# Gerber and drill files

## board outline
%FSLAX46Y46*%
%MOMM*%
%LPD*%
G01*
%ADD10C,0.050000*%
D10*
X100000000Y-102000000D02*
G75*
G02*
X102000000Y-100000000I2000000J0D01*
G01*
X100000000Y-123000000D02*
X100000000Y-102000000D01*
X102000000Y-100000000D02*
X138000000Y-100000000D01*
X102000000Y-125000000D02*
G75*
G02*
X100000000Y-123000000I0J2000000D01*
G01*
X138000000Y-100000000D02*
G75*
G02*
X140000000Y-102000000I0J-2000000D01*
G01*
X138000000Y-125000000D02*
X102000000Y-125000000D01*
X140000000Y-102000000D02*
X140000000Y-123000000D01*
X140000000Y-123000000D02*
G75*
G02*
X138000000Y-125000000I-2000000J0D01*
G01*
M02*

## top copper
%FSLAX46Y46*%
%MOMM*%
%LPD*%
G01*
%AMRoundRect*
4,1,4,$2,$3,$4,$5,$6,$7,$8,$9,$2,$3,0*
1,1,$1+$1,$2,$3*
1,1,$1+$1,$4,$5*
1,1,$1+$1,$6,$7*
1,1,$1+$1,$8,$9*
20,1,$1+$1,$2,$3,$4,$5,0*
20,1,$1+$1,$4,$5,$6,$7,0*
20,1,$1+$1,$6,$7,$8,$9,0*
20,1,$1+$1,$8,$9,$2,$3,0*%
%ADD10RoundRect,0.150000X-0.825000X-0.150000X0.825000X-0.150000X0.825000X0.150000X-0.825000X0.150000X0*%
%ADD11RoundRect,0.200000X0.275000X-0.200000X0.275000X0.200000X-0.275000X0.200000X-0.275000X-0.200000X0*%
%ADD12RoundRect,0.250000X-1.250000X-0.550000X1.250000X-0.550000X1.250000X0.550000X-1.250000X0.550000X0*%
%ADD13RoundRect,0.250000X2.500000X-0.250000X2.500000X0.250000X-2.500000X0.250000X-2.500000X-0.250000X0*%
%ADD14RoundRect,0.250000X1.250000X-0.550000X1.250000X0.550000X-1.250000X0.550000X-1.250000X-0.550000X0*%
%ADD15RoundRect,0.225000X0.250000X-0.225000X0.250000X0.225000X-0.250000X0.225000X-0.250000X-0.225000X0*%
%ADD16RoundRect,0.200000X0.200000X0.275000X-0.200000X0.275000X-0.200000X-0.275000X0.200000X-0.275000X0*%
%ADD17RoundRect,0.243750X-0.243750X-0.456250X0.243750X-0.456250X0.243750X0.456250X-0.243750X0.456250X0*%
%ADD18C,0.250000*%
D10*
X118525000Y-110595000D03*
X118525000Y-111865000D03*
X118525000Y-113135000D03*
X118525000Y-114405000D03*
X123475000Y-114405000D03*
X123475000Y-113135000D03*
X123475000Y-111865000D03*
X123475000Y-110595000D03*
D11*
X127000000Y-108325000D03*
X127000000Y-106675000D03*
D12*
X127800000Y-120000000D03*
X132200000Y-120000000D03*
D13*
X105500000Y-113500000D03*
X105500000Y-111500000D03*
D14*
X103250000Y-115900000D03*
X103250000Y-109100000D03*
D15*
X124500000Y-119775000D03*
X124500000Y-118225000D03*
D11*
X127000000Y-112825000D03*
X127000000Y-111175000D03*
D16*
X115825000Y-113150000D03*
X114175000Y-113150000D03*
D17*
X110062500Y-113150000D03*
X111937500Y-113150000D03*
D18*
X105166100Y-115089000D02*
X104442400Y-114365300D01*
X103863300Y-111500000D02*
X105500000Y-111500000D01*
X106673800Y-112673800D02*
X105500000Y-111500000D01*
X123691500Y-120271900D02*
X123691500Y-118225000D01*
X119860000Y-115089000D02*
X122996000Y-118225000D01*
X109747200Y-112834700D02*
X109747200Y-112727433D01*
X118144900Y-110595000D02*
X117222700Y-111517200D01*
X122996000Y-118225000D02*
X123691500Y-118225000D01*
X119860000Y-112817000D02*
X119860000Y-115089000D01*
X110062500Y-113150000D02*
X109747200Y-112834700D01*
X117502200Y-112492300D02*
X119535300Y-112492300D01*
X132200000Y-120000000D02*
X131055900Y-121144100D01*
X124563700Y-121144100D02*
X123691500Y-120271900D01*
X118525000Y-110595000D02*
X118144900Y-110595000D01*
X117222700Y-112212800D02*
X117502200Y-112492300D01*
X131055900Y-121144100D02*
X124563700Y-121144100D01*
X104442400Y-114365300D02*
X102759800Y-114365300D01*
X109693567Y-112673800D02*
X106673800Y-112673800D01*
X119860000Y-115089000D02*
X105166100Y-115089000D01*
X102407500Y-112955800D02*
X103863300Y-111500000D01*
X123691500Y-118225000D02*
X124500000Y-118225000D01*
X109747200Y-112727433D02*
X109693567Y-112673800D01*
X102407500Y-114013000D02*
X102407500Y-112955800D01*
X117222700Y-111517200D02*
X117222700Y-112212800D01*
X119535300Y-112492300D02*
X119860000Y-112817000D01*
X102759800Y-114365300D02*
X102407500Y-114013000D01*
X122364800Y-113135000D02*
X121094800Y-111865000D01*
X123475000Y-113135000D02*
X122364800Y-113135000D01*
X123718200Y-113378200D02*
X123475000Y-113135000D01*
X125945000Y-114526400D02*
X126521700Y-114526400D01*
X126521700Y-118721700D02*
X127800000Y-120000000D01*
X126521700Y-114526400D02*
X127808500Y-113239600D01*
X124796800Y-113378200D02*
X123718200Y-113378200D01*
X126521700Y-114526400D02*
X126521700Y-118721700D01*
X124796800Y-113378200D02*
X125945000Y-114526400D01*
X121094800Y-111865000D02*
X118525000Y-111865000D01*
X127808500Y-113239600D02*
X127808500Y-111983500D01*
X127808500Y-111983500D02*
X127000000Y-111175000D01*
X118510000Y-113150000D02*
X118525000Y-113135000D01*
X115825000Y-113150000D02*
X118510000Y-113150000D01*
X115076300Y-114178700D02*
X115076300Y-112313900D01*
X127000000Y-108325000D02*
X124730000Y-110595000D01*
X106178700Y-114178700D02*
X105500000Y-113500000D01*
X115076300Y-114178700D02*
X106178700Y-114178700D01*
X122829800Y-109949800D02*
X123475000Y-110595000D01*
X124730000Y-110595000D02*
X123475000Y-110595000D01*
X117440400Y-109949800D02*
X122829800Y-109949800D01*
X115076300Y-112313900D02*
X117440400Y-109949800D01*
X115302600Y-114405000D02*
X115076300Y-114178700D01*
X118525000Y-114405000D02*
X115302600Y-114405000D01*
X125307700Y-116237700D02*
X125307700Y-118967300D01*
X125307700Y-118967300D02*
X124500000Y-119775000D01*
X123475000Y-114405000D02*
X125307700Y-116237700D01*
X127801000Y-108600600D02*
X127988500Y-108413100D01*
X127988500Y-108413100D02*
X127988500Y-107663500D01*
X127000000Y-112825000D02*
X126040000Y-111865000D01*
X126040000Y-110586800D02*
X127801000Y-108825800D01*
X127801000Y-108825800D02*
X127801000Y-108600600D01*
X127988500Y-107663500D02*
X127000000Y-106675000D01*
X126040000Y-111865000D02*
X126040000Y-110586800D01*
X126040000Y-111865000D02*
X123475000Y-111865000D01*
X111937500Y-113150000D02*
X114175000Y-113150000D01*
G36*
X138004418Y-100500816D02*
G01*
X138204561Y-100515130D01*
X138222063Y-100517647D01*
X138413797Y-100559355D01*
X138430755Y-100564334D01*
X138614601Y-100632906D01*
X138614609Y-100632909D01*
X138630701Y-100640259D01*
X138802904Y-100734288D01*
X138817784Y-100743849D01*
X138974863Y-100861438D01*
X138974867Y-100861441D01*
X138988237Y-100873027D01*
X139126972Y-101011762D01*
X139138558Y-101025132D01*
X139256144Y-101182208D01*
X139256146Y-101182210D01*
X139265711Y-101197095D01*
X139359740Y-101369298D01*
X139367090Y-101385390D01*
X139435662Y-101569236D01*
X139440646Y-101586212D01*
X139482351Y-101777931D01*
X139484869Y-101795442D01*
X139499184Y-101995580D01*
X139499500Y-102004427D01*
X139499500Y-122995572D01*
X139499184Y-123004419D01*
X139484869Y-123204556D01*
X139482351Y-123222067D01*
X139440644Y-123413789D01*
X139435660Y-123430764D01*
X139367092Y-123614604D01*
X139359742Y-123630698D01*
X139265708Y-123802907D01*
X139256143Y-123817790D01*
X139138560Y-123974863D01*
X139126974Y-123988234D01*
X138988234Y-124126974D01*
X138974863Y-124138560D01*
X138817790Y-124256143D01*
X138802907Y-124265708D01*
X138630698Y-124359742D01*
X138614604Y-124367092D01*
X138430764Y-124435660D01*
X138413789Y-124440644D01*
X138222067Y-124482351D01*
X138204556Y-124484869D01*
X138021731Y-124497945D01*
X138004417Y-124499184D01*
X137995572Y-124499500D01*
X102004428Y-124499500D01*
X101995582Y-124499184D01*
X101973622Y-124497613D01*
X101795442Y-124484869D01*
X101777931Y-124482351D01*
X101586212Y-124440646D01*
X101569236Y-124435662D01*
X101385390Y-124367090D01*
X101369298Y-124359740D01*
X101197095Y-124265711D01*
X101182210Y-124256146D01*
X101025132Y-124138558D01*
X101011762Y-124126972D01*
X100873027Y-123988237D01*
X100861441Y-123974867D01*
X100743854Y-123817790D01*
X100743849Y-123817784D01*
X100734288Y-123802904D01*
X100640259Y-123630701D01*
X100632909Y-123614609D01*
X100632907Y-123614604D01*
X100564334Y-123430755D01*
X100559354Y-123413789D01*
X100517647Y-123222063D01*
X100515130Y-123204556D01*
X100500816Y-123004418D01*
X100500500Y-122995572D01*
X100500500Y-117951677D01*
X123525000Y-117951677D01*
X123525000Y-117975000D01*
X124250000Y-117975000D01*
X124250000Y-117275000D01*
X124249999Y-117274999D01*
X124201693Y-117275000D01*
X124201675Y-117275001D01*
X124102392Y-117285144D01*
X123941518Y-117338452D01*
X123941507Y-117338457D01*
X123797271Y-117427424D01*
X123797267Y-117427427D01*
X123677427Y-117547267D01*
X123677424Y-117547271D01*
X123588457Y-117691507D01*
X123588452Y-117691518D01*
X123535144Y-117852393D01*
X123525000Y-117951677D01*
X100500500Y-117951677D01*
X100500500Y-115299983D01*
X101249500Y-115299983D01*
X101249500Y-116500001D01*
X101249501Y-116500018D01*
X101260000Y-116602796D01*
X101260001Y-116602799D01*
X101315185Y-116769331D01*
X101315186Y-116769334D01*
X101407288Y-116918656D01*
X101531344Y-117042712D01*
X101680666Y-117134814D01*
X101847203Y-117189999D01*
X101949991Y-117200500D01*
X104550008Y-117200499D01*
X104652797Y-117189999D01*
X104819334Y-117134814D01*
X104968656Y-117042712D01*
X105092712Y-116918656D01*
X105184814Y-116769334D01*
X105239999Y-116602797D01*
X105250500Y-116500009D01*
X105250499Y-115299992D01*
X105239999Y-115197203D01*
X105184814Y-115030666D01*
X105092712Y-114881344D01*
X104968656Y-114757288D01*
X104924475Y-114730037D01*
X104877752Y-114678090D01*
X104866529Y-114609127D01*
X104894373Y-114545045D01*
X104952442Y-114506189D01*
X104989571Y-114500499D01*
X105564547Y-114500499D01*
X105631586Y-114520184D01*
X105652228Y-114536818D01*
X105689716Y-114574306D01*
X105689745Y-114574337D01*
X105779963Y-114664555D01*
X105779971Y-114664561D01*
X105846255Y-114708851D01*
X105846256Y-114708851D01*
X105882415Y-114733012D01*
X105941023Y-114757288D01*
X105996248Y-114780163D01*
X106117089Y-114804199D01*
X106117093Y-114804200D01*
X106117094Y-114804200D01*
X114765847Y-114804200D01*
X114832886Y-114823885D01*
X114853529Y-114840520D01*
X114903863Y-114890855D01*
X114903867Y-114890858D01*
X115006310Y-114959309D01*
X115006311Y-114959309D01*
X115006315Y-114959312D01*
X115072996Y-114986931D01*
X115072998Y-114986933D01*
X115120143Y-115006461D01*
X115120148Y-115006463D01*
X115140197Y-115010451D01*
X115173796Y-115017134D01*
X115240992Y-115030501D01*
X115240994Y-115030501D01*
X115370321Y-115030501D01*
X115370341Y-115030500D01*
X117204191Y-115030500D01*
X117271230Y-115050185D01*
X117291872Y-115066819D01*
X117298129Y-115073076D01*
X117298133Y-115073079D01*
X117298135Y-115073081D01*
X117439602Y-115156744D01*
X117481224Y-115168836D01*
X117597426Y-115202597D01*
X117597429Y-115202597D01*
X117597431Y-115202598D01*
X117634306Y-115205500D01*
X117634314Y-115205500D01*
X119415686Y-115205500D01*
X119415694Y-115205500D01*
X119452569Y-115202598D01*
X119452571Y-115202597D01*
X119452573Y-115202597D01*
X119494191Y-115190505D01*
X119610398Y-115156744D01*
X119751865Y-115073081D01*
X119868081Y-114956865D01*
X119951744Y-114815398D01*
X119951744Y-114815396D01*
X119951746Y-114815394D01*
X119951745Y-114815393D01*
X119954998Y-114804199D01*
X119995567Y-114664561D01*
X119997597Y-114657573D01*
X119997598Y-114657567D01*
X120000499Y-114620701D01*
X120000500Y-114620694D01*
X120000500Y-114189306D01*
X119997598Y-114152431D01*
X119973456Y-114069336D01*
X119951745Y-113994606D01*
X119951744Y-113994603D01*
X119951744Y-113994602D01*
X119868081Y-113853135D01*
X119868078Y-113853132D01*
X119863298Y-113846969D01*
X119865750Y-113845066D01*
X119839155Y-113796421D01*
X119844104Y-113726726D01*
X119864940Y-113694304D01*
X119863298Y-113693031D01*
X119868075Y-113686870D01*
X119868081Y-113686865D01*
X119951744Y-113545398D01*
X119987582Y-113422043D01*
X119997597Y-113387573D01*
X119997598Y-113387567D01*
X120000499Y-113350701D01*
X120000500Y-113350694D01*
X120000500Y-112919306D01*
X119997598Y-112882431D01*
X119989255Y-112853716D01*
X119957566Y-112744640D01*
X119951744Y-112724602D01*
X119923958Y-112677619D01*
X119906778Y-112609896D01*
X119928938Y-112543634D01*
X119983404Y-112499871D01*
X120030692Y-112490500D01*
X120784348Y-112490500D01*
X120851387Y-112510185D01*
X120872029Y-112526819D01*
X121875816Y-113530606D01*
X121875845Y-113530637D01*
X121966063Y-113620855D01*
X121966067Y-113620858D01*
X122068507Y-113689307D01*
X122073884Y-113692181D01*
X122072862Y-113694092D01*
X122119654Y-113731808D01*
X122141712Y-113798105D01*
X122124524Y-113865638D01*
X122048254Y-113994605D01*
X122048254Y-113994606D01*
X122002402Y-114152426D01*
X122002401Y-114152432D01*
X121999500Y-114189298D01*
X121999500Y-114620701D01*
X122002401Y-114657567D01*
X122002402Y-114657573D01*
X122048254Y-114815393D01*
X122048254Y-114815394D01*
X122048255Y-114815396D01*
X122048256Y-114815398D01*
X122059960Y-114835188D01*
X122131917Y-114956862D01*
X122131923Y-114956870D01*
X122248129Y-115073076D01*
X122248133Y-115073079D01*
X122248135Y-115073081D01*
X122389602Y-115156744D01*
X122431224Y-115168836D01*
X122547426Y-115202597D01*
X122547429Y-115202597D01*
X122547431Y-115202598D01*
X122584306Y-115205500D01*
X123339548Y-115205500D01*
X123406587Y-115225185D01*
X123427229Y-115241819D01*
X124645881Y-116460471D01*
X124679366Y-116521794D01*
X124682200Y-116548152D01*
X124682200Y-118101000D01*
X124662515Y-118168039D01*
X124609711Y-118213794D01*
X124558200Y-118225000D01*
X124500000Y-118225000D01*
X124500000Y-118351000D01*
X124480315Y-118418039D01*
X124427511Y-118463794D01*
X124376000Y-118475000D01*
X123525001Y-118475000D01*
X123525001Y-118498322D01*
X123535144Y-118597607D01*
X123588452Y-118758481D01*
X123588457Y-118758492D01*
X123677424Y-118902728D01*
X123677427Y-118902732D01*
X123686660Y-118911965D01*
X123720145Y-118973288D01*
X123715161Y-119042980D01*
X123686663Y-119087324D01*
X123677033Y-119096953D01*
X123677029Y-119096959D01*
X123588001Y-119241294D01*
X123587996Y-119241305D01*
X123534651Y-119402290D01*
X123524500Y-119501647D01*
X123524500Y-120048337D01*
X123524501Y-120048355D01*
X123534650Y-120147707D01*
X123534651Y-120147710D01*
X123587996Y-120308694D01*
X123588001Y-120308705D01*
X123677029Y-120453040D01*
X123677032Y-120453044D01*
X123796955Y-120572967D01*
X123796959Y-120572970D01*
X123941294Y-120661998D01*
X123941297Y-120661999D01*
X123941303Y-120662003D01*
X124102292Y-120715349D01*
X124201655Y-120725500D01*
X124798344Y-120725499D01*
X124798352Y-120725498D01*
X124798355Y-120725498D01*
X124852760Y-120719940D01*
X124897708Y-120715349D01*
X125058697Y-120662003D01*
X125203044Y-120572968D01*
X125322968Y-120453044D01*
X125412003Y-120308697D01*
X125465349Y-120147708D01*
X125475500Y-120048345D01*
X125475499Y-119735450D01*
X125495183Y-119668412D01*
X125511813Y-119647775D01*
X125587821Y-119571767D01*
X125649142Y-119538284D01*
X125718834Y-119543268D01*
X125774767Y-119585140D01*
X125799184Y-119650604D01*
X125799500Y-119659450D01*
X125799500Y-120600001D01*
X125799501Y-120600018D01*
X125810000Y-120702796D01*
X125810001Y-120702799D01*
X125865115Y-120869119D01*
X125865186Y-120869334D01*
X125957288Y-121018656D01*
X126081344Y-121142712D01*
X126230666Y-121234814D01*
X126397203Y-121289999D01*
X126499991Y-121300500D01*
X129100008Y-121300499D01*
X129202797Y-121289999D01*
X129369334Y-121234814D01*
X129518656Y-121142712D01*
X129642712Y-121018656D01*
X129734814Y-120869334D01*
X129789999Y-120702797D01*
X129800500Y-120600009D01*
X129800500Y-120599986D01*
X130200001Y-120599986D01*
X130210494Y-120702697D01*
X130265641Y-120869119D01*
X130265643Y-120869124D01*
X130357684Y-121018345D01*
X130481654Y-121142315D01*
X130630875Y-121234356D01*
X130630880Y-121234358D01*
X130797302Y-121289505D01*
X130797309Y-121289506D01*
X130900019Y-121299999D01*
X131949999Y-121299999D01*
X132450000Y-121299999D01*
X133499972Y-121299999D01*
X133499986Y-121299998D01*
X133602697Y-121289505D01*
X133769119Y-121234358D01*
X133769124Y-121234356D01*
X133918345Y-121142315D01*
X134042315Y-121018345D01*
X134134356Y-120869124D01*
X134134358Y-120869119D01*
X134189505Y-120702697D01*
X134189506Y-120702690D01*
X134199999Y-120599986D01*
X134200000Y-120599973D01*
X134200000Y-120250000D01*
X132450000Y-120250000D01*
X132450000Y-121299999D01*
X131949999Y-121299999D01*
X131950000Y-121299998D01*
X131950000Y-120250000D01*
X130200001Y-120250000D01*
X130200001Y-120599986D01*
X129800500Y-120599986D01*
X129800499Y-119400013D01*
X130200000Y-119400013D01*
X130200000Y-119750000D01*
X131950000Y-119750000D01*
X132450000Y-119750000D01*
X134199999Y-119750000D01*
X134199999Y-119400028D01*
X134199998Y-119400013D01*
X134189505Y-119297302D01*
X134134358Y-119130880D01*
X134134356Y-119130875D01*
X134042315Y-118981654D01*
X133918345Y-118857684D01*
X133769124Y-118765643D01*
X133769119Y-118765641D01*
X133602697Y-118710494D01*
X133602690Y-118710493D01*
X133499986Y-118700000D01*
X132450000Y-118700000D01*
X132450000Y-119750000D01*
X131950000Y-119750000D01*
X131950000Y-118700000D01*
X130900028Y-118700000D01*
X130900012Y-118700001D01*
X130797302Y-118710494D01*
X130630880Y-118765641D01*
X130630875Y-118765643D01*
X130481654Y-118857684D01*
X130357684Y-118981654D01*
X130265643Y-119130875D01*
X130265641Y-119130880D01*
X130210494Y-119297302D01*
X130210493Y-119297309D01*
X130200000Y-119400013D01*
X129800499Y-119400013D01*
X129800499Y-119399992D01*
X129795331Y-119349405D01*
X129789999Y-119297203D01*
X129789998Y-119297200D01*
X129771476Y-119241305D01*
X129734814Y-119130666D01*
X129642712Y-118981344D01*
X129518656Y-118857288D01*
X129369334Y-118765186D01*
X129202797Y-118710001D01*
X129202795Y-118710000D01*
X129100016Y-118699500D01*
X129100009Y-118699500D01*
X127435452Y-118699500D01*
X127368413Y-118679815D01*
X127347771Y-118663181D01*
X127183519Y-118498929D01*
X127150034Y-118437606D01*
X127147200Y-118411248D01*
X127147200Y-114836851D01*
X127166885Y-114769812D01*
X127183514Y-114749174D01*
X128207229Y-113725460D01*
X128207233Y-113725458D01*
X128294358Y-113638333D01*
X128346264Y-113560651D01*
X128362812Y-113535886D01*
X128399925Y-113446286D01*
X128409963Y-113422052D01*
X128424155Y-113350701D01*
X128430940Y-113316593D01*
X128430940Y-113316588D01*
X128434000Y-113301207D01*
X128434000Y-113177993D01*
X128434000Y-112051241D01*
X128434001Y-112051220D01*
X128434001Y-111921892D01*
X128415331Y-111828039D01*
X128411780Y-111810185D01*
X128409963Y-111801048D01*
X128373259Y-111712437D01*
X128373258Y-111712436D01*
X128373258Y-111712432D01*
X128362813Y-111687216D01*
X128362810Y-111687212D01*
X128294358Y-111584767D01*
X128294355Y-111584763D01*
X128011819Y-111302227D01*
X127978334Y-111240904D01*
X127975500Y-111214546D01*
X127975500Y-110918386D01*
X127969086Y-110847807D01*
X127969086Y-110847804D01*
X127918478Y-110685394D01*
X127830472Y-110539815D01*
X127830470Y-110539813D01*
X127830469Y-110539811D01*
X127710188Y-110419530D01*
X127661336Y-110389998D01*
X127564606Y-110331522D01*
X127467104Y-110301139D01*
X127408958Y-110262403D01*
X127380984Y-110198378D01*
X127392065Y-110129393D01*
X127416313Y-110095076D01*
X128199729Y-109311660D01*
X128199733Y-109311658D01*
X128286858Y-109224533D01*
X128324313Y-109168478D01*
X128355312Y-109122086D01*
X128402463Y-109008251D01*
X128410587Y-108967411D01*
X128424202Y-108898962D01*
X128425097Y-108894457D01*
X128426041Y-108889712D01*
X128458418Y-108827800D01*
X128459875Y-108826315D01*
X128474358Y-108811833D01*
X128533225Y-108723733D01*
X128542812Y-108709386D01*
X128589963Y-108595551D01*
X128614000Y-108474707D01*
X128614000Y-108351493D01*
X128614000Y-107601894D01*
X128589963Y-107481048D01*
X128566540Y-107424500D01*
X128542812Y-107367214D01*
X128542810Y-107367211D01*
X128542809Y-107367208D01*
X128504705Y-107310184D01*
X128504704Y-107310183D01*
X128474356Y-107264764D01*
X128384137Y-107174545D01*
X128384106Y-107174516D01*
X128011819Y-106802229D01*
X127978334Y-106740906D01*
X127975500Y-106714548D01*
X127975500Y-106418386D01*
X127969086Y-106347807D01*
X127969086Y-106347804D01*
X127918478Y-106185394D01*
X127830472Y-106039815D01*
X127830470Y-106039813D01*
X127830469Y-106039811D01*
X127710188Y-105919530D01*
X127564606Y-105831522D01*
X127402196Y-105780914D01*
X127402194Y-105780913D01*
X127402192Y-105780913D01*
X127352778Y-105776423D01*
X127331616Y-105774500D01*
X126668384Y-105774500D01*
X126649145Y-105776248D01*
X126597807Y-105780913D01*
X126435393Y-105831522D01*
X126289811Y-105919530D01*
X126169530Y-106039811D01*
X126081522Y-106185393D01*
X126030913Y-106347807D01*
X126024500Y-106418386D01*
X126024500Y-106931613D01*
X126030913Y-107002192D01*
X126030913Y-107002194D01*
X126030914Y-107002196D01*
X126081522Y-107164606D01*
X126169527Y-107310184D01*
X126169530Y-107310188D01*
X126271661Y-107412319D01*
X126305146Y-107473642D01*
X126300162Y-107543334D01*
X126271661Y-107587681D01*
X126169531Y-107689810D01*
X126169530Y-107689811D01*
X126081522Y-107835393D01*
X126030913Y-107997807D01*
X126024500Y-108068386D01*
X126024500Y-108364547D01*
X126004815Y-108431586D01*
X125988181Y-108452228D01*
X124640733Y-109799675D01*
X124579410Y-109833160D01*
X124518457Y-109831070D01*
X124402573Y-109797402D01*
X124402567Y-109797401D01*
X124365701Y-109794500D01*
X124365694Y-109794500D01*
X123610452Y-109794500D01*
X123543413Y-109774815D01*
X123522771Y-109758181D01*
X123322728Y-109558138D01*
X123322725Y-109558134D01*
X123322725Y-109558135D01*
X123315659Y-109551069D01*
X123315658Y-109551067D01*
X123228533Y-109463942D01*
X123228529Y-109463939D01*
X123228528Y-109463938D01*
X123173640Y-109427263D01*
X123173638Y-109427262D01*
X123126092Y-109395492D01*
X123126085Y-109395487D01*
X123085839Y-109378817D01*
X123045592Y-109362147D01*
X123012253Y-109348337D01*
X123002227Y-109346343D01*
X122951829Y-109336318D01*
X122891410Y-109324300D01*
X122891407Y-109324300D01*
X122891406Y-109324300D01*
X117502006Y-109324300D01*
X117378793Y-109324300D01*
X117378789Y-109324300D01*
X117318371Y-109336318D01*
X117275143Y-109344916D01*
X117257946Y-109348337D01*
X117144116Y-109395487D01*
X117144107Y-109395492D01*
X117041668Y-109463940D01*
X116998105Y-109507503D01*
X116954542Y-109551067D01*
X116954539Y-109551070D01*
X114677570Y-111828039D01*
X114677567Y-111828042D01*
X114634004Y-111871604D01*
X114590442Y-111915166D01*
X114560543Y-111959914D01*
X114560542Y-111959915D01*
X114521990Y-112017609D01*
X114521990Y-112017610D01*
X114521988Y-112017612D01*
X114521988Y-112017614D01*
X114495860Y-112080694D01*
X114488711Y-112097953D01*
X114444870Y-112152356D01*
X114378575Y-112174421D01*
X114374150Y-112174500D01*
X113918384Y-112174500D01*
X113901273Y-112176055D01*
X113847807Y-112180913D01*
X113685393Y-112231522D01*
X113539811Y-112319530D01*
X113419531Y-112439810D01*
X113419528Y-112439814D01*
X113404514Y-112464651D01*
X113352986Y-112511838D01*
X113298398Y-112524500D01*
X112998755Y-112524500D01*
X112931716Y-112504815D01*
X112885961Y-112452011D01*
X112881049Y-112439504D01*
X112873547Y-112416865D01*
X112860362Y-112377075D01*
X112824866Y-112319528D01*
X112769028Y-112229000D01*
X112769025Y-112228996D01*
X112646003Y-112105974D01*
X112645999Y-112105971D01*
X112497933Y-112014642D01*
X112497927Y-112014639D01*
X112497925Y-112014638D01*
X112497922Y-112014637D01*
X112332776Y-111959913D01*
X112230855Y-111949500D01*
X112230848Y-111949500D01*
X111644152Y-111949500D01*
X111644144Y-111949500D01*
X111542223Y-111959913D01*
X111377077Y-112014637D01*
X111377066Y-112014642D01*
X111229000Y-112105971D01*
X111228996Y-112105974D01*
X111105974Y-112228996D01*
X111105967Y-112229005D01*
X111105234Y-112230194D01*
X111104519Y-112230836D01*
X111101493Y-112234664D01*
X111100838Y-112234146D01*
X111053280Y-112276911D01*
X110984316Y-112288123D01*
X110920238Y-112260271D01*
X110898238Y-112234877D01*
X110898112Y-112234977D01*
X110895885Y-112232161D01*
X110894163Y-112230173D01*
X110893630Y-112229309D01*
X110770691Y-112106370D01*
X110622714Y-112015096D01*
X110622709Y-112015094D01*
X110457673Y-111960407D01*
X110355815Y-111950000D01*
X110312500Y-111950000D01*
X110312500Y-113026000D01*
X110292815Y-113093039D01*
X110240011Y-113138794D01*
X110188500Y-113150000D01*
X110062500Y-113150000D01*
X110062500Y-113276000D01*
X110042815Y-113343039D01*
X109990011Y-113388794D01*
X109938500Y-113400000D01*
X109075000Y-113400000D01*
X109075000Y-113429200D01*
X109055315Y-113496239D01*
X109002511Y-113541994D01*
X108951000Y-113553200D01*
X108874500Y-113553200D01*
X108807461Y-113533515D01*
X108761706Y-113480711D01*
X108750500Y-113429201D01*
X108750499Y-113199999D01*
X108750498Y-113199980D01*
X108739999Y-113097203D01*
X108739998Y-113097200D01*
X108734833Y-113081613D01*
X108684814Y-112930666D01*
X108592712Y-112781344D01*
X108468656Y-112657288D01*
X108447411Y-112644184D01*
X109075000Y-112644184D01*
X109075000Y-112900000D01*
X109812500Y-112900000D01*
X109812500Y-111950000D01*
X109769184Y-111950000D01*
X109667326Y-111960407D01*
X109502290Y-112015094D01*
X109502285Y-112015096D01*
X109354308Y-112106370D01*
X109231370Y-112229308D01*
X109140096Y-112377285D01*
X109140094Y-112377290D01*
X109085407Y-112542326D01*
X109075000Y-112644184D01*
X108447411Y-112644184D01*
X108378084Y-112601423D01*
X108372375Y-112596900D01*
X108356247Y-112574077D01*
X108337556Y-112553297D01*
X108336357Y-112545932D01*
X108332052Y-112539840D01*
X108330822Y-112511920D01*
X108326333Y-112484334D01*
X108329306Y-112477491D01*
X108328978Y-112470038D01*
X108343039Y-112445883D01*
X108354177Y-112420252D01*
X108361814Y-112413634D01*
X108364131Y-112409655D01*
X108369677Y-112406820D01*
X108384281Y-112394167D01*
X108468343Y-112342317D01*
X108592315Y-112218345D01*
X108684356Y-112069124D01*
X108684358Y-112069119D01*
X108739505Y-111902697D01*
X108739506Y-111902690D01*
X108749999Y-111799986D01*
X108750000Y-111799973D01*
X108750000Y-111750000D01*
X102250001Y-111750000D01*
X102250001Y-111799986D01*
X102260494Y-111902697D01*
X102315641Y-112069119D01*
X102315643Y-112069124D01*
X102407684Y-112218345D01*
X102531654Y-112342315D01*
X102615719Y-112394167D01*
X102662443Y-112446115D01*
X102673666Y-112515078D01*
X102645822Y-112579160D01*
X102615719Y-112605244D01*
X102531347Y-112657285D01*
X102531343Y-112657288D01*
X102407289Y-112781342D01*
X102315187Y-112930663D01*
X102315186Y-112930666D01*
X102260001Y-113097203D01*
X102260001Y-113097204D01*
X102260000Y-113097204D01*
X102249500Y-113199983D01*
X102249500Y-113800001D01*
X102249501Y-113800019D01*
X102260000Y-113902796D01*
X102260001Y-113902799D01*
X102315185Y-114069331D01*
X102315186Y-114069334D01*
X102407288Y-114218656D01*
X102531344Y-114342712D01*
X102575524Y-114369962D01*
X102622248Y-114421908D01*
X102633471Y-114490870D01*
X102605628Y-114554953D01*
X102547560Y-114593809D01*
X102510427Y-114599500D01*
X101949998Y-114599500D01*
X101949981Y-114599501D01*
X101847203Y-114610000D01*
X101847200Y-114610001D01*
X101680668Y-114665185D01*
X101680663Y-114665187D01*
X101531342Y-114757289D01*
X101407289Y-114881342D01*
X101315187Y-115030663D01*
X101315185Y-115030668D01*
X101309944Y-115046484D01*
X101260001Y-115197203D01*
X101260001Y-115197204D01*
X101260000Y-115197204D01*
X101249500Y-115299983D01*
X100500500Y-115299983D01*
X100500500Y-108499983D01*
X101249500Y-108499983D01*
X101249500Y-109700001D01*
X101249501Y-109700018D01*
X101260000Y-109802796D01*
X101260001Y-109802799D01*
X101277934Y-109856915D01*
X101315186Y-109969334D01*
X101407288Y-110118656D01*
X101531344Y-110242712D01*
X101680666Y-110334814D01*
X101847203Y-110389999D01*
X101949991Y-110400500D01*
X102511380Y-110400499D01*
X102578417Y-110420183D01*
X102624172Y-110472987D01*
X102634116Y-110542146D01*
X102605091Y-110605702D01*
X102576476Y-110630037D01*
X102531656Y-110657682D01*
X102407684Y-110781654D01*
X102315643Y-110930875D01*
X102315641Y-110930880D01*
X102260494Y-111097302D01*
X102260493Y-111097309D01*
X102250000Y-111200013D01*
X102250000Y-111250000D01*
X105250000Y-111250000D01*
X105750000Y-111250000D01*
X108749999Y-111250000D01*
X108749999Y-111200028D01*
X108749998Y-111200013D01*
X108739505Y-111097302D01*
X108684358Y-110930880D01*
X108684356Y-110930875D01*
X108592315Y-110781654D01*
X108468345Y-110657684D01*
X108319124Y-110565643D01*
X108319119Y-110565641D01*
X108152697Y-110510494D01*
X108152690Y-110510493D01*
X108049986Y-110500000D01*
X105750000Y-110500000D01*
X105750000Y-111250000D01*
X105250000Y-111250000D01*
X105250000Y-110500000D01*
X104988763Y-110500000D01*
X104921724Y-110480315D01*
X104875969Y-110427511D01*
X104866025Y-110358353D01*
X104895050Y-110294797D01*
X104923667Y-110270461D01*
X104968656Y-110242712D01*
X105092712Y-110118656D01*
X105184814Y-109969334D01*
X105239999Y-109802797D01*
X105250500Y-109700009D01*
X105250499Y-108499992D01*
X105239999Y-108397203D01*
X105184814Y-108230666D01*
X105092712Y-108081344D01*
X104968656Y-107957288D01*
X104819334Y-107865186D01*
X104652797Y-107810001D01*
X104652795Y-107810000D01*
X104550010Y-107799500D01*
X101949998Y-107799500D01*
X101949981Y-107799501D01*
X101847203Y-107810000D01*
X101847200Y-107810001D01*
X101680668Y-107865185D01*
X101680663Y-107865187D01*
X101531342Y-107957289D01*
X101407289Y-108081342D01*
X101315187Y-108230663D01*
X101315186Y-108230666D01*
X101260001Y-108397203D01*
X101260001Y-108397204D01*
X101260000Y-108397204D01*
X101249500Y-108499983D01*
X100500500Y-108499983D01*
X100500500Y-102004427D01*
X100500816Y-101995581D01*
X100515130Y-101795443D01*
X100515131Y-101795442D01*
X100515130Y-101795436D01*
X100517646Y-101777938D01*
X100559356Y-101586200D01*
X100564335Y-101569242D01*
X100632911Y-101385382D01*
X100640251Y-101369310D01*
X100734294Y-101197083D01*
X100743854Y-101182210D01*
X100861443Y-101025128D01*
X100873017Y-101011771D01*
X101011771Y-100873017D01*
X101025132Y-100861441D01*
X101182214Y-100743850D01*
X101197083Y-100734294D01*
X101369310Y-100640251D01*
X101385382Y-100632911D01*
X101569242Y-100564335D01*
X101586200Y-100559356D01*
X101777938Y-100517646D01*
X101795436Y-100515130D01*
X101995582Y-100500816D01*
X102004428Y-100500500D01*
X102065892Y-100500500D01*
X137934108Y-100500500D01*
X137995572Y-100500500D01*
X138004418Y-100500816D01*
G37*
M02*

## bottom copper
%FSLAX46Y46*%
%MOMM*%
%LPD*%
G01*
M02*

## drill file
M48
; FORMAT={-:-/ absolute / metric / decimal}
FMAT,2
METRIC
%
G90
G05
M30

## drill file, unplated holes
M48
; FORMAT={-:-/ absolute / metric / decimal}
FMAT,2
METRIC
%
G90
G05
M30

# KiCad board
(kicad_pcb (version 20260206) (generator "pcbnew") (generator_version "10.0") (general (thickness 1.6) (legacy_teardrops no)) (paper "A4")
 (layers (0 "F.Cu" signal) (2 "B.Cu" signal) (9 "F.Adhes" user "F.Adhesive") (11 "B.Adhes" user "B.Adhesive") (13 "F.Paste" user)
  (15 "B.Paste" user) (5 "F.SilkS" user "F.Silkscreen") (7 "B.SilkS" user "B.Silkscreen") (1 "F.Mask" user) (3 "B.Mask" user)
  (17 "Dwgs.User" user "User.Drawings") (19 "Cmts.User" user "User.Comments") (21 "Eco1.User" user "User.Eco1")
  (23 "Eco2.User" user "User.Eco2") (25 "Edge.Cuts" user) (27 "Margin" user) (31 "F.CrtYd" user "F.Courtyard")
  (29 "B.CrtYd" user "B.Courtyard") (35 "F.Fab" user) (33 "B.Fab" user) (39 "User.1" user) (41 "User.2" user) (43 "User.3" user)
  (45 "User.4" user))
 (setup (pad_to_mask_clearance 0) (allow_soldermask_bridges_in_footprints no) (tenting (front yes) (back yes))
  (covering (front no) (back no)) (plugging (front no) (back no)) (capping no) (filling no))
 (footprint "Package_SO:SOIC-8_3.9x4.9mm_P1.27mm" (layer "F.Cu") (at 121 112.5)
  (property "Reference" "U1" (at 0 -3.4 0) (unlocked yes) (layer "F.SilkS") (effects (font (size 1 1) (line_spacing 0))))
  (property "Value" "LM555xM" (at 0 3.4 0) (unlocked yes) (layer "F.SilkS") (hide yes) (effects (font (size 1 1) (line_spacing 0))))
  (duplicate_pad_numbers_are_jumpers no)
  (pad "1" smd roundrect (at -2.475 -1.905) (size 1.95 0.6) (layers "F.Cu" "F.Mask" "F.Paste") (roundrect_rratio 0.25) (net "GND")
   (zone_connect 0))
  (pad "2" smd roundrect (at -2.475 -0.635) (size 1.95 0.6) (layers "F.Cu" "F.Mask" "F.Paste") (roundrect_rratio 0.25)
   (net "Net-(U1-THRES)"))
  (pad "3" smd roundrect (at -2.475 0.635) (size 1.95 0.6) (layers "F.Cu" "F.Mask" "F.Paste") (roundrect_rratio 0.25) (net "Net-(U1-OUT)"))
  (pad "4" smd roundrect (at -2.475 1.905) (size 1.95 0.6) (layers "F.Cu" "F.Mask" "F.Paste") (roundrect_rratio 0.25) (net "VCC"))
  (pad "5" smd roundrect (at 2.475 1.905) (size 1.95 0.6) (layers "F.Cu" "F.Mask" "F.Paste") (roundrect_rratio 0.25) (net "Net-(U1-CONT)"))
  (pad "6" smd roundrect (at 2.475 0.635) (size 1.95 0.6) (layers "F.Cu" "F.Mask" "F.Paste") (roundrect_rratio 0.25) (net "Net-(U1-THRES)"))
  (pad "7" smd roundrect (at 2.475 -0.635) (size 1.95 0.6) (layers "F.Cu" "F.Mask" "F.Paste") (roundrect_rratio 0.25) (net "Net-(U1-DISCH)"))
  (pad "8" smd roundrect (at 2.475 -1.905) (size 1.95 0.6) (layers "F.Cu" "F.Mask" "F.Paste") (roundrect_rratio 0.25) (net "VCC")))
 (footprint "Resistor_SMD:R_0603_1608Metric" (layer "F.Cu") (at 127 107.5 90)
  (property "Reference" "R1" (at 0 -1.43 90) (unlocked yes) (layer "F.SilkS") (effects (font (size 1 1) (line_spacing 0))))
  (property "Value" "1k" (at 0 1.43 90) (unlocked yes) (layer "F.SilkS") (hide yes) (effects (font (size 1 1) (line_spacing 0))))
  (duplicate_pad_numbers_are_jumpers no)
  (pad "1" smd roundrect (at -0.825 0 90) (size 0.8 0.95) (layers "F.Cu" "F.Mask" "F.Paste") (roundrect_rratio 0.25) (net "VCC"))
  (pad "2" smd roundrect (at 0.825 0 90) (size 0.8 0.95) (layers "F.Cu" "F.Mask" "F.Paste") (roundrect_rratio 0.25) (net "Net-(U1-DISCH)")))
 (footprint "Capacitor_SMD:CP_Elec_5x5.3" (layer "F.Cu") (at 130 120)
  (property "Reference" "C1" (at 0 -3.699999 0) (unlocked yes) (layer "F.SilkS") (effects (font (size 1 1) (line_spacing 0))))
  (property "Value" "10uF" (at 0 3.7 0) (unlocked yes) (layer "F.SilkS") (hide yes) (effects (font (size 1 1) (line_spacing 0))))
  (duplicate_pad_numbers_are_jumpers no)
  (pad "1" smd roundrect (at -2.2 0) (size 3 1.6) (layers "F.Cu" "F.Mask" "F.Paste") (roundrect_rratio 0.15625) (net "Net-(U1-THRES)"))
  (pad "2" smd roundrect (at 2.2 0) (size 3 1.6) (layers "F.Cu" "F.Mask" "F.Paste") (roundrect_rratio 0.15625) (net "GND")))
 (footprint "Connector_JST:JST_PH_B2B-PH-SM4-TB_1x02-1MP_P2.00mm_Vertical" (layer "F.Cu") (at 105 112.5 90)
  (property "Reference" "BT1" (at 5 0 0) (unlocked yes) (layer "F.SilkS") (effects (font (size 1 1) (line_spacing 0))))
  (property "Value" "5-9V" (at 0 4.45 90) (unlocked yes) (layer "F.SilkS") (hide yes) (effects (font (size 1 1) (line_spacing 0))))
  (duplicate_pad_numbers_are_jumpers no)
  (pad "1" smd roundrect (at -1 0.5 90) (size 1 5.5) (layers "F.Cu" "F.Mask" "F.Paste") (roundrect_rratio 0.25) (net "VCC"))
  (pad "2" smd roundrect (at 1 0.5 90) (size 1 5.5) (layers "F.Cu" "F.Mask" "F.Paste") (roundrect_rratio 0.25) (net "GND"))
  (pad "MP" smd roundrect (at -3.4 -1.75 90) (size 1.6 3) (layers "F.Cu" "F.Mask" "F.Paste") (roundrect_rratio 0.15625))
  (pad "MP" smd roundrect (at 3.4 -1.75 90) (size 1.6 3) (layers "F.Cu" "F.Mask" "F.Paste") (roundrect_rratio 0.15625)))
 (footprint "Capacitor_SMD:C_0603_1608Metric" (layer "F.Cu") (at 124.5 119 90)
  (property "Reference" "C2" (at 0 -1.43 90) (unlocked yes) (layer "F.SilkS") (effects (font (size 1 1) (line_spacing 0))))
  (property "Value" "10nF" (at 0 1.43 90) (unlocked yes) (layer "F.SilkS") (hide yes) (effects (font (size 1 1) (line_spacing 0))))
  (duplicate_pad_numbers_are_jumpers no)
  (pad "1" smd roundrect (at -0.775 0 90) (size 0.9 0.95) (layers "F.Cu" "F.Mask" "F.Paste") (roundrect_rratio 0.25) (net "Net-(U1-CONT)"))
  (pad "2" smd roundrect (at 0.775 0 90) (size 0.9 0.95) (layers "F.Cu" "F.Mask" "F.Paste") (roundrect_rratio 0.25) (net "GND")))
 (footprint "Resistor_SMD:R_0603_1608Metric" (layer "F.Cu") (at 127 112 90)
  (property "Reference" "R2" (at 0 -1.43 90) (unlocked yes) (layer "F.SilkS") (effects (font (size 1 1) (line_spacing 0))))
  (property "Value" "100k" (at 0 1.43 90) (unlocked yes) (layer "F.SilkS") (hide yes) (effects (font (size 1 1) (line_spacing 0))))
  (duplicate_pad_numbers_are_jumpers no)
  (pad "1" smd roundrect (at -0.825 0 90) (size 0.8 0.95) (layers "F.Cu" "F.Mask" "F.Paste") (roundrect_rratio 0.25) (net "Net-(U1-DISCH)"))
  (pad "2" smd roundrect (at 0.825 0 90) (size 0.8 0.95) (layers "F.Cu" "F.Mask" "F.Paste") (roundrect_rratio 0.25) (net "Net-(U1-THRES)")))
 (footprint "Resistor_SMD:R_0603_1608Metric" (layer "F.Cu") (at 115 113.15 180)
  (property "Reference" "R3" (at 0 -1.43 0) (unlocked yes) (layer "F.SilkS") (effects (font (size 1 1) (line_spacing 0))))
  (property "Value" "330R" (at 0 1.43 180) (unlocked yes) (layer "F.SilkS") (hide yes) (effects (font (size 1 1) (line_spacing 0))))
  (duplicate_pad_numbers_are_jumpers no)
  (pad "1" smd roundrect (at -0.825 0 180) (size 0.8 0.95) (layers "F.Cu" "F.Mask" "F.Paste") (roundrect_rratio 0.25) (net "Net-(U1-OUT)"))
  (pad "2" smd roundrect (at 0.825 0 180) (size 0.8 0.95) (layers "F.Cu" "F.Mask" "F.Paste") (roundrect_rratio 0.25) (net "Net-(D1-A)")))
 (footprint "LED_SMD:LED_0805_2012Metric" (layer "F.Cu") (at 111 113.15)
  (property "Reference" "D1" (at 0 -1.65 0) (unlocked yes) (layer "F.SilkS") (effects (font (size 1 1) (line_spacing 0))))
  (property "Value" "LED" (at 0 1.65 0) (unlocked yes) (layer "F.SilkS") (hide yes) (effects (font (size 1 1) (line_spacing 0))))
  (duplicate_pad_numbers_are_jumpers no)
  (pad "1" smd roundrect (at -0.9375 0) (size 0.975 1.4) (layers "F.Cu" "F.Mask" "F.Paste") (roundrect_rratio 0.25) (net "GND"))
  (pad "2" smd roundrect (at 0.9375 0) (size 0.975 1.4) (layers "F.Cu" "F.Mask" "F.Paste") (roundrect_rratio 0.25) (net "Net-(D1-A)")))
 (gr_arc (start 100 102) (mid 100.585786 100.585786) (end 102 100) (stroke (width 0.05) (type default)) (layer "Edge.Cuts"))
 (gr_line (start 100 123) (end 100 102) (stroke (width 0.05) (type default)) (layer "Edge.Cuts"))
 (gr_line (start 102 100) (end 138 100) (stroke (width 0.05) (type default)) (layer "Edge.Cuts"))
 (gr_arc (start 102 125) (mid 100.585786 124.414213) (end 100 123) (stroke (width 0.05) (type default)) (layer "Edge.Cuts"))
 (gr_arc (start 138 100) (mid 139.414213 100.585786) (end 140 102) (stroke (width 0.05) (type default)) (layer "Edge.Cuts"))
 (gr_line (start 138 125) (end 102 125) (stroke (width 0.05) (type default)) (layer "Edge.Cuts"))
 (gr_line (start 140 102) (end 140 123) (stroke (width 0.05) (type default)) (layer "Edge.Cuts"))
 (gr_arc (start 140 123) (mid 139.414213 124.414213) (end 138 125) (stroke (width 0.05) (type default)) (layer "Edge.Cuts"))
 (segment (start 105.1661 115.089) (end 104.4424 114.3653) (width 0.25) (layer "F.Cu") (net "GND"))
 (segment (start 103.8633 111.5) (end 105.5 111.5) (width 0.25) (layer "F.Cu") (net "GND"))
 (segment (start 106.6738 112.6738) (end 105.5 111.5) (width 0.25) (layer "F.Cu") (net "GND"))
 (segment (start 123.6915 120.2719) (end 123.6915 118.225) (width 0.25) (layer "F.Cu") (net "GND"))
 (segment (start 119.86 115.089) (end 122.996 118.225) (width 0.25) (layer "F.Cu") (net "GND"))
 (segment (start 109.7472 112.8347) (end 109.747200 112.727433) (width 0.25) (layer "F.Cu") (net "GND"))
 (segment (start 118.1449 110.595) (end 117.2227 111.5172) (width 0.25) (layer "F.Cu") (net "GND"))
 (segment (start 122.996 118.225) (end 123.6915 118.225) (width 0.25) (layer "F.Cu") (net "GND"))
 (segment (start 119.86 112.817) (end 119.86 115.089) (width 0.25) (layer "F.Cu") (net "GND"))
 (segment (start 110.0625 113.15) (end 109.7472 112.8347) (width 0.25) (layer "F.Cu") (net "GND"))
 (segment (start 117.5022 112.4923) (end 119.5353 112.4923) (width 0.25) (layer "F.Cu") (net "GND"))
 (segment (start 132.2 120) (end 131.0559 121.1441) (width 0.25) (layer "F.Cu") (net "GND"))
 (segment (start 124.5637 121.1441) (end 123.6915 120.2719) (width 0.25) (layer "F.Cu") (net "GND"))
 (segment (start 118.525 110.595) (end 118.1449 110.595) (width 0.25) (layer "F.Cu") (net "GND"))
 (segment (start 117.2227 112.2128) (end 117.5022 112.4923) (width 0.25) (layer "F.Cu") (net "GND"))
 (segment (start 131.0559 121.1441) (end 124.5637 121.1441) (width 0.25) (layer "F.Cu") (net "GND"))
 (segment (start 104.4424 114.3653) (end 102.7598 114.3653) (width 0.25) (layer "F.Cu") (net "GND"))
 (segment (start 109.693567 112.673800) (end 106.6738 112.6738) (width 0.25) (layer "F.Cu") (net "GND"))
 (segment (start 119.86 115.089) (end 105.1661 115.089) (width 0.25) (layer "F.Cu") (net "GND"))
 (segment (start 102.4075 112.9558) (end 103.8633 111.5) (width 0.25) (layer "F.Cu") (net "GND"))
 (segment (start 123.6915 118.225) (end 124.5 118.225) (width 0.25) (layer "F.Cu") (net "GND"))
 (segment (start 102.4075 114.013) (end 102.4075 112.9558) (width 0.25) (layer "F.Cu") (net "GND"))
 (segment (start 117.2227 111.5172) (end 117.2227 112.2128) (width 0.25) (layer "F.Cu") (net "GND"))
 (segment (start 119.5353 112.4923) (end 119.86 112.817) (width 0.25) (layer "F.Cu") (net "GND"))
 (segment (start 102.7598 114.3653) (end 102.4075 114.013) (width 0.25) (layer "F.Cu") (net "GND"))
 (segment (start 122.3648 113.135) (end 121.0948 111.865) (width 0.25) (layer "F.Cu") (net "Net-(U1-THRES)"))
 (segment (start 123.475 113.135) (end 122.3648 113.135) (width 0.25) (layer "F.Cu") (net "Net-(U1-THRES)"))
 (segment (start 123.7182 113.3782) (end 123.475 113.135) (width 0.25) (layer "F.Cu") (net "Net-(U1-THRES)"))
 (segment (start 125.945 114.5264) (end 126.5217 114.5264) (width 0.25) (layer "F.Cu") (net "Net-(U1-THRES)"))
 (segment (start 126.5217 118.7217) (end 127.8 120) (width 0.25) (layer "F.Cu") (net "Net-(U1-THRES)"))
 (segment (start 126.5217 114.5264) (end 127.8085 113.2396) (width 0.25) (layer "F.Cu") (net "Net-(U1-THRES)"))
 (segment (start 124.7968 113.3782) (end 123.7182 113.3782) (width 0.25) (layer "F.Cu") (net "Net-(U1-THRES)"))
 (segment (start 126.5217 114.5264) (end 126.5217 118.7217) (width 0.25) (layer "F.Cu") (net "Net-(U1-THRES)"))
 (segment (start 124.7968 113.3782) (end 125.945 114.5264) (width 0.25) (layer "F.Cu") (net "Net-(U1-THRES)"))
 (segment (start 121.0948 111.865) (end 118.525 111.865) (width 0.25) (layer "F.Cu") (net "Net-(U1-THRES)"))
 (segment (start 127.8085 113.2396) (end 127.8085 111.9835) (width 0.25) (layer "F.Cu") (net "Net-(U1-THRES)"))
 (segment (start 127.8085 111.9835) (end 127 111.175) (width 0.25) (layer "F.Cu") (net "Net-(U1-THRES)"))
 (segment (start 118.51 113.15) (end 118.525 113.135) (width 0.25) (layer "F.Cu") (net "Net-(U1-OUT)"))
 (segment (start 115.825 113.15) (end 118.51 113.15) (width 0.25) (layer "F.Cu") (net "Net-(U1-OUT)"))
 (segment (start 115.0763 114.1787) (end 115.0763 112.3139) (width 0.25) (layer "F.Cu") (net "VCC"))
 (segment (start 127 108.325) (end 124.73 110.595) (width 0.25) (layer "F.Cu") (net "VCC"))
 (segment (start 106.1787 114.1787) (end 105.5 113.5) (width 0.25) (layer "F.Cu") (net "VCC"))
 (segment (start 115.0763 114.1787) (end 106.1787 114.1787) (width 0.25) (layer "F.Cu") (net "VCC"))
 (segment (start 122.8298 109.9498) (end 123.475 110.595) (width 0.25) (layer "F.Cu") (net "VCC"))
 (segment (start 124.73 110.595) (end 123.475 110.595) (width 0.25) (layer "F.Cu") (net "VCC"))
 (segment (start 117.4404 109.9498) (end 122.8298 109.9498) (width 0.25) (layer "F.Cu") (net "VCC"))
 (segment (start 115.0763 112.3139) (end 117.4404 109.9498) (width 0.25) (layer "F.Cu") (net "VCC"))
 (segment (start 115.3026 114.405) (end 115.0763 114.1787) (width 0.25) (layer "F.Cu") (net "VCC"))
 (segment (start 118.525 114.405) (end 115.3026 114.405) (width 0.25) (layer "F.Cu") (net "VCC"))
 (segment (start 125.3077 116.2377) (end 125.3077 118.9673) (width 0.25) (layer "F.Cu") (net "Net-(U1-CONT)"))
 (segment (start 125.3077 118.9673) (end 124.5 119.775) (width 0.25) (layer "F.Cu") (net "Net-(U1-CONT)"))
 (segment (start 123.475 114.405) (end 125.3077 116.2377) (width 0.25) (layer "F.Cu") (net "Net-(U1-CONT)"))
 (segment (start 127.801 108.6006) (end 127.9885 108.4131) (width 0.25) (layer "F.Cu") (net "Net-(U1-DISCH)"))
 (segment (start 127.9885 108.4131) (end 127.9885 107.6635) (width 0.25) (layer "F.Cu") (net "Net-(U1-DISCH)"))
 (segment (start 127 112.825) (end 126.04 111.865) (width 0.25) (layer "F.Cu") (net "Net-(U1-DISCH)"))
 (segment (start 126.04 110.5868) (end 127.801 108.8258) (width 0.25) (layer "F.Cu") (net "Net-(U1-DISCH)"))
 (segment (start 127.801 108.8258) (end 127.801 108.6006) (width 0.25) (layer "F.Cu") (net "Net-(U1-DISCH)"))
 (segment (start 127.9885 107.6635) (end 127 106.675) (width 0.25) (layer "F.Cu") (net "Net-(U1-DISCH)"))
 (segment (start 126.04 111.865) (end 126.04 110.5868) (width 0.25) (layer "F.Cu") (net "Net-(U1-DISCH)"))
 (segment (start 126.04 111.865) (end 123.475 111.865) (width 0.25) (layer "F.Cu") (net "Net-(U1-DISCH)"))
 (segment (start 111.9375 113.15) (end 114.175 113.15) (width 0.25) (layer "F.Cu") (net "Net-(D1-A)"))
 (segment (start 109.747200 112.727433) (end 109.693567 112.673800) (width 0.25) (layer "F.Cu") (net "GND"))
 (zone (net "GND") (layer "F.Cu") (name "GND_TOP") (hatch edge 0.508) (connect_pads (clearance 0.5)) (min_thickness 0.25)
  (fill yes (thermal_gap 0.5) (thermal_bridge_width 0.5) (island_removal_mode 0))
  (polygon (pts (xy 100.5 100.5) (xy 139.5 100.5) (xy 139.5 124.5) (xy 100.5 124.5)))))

